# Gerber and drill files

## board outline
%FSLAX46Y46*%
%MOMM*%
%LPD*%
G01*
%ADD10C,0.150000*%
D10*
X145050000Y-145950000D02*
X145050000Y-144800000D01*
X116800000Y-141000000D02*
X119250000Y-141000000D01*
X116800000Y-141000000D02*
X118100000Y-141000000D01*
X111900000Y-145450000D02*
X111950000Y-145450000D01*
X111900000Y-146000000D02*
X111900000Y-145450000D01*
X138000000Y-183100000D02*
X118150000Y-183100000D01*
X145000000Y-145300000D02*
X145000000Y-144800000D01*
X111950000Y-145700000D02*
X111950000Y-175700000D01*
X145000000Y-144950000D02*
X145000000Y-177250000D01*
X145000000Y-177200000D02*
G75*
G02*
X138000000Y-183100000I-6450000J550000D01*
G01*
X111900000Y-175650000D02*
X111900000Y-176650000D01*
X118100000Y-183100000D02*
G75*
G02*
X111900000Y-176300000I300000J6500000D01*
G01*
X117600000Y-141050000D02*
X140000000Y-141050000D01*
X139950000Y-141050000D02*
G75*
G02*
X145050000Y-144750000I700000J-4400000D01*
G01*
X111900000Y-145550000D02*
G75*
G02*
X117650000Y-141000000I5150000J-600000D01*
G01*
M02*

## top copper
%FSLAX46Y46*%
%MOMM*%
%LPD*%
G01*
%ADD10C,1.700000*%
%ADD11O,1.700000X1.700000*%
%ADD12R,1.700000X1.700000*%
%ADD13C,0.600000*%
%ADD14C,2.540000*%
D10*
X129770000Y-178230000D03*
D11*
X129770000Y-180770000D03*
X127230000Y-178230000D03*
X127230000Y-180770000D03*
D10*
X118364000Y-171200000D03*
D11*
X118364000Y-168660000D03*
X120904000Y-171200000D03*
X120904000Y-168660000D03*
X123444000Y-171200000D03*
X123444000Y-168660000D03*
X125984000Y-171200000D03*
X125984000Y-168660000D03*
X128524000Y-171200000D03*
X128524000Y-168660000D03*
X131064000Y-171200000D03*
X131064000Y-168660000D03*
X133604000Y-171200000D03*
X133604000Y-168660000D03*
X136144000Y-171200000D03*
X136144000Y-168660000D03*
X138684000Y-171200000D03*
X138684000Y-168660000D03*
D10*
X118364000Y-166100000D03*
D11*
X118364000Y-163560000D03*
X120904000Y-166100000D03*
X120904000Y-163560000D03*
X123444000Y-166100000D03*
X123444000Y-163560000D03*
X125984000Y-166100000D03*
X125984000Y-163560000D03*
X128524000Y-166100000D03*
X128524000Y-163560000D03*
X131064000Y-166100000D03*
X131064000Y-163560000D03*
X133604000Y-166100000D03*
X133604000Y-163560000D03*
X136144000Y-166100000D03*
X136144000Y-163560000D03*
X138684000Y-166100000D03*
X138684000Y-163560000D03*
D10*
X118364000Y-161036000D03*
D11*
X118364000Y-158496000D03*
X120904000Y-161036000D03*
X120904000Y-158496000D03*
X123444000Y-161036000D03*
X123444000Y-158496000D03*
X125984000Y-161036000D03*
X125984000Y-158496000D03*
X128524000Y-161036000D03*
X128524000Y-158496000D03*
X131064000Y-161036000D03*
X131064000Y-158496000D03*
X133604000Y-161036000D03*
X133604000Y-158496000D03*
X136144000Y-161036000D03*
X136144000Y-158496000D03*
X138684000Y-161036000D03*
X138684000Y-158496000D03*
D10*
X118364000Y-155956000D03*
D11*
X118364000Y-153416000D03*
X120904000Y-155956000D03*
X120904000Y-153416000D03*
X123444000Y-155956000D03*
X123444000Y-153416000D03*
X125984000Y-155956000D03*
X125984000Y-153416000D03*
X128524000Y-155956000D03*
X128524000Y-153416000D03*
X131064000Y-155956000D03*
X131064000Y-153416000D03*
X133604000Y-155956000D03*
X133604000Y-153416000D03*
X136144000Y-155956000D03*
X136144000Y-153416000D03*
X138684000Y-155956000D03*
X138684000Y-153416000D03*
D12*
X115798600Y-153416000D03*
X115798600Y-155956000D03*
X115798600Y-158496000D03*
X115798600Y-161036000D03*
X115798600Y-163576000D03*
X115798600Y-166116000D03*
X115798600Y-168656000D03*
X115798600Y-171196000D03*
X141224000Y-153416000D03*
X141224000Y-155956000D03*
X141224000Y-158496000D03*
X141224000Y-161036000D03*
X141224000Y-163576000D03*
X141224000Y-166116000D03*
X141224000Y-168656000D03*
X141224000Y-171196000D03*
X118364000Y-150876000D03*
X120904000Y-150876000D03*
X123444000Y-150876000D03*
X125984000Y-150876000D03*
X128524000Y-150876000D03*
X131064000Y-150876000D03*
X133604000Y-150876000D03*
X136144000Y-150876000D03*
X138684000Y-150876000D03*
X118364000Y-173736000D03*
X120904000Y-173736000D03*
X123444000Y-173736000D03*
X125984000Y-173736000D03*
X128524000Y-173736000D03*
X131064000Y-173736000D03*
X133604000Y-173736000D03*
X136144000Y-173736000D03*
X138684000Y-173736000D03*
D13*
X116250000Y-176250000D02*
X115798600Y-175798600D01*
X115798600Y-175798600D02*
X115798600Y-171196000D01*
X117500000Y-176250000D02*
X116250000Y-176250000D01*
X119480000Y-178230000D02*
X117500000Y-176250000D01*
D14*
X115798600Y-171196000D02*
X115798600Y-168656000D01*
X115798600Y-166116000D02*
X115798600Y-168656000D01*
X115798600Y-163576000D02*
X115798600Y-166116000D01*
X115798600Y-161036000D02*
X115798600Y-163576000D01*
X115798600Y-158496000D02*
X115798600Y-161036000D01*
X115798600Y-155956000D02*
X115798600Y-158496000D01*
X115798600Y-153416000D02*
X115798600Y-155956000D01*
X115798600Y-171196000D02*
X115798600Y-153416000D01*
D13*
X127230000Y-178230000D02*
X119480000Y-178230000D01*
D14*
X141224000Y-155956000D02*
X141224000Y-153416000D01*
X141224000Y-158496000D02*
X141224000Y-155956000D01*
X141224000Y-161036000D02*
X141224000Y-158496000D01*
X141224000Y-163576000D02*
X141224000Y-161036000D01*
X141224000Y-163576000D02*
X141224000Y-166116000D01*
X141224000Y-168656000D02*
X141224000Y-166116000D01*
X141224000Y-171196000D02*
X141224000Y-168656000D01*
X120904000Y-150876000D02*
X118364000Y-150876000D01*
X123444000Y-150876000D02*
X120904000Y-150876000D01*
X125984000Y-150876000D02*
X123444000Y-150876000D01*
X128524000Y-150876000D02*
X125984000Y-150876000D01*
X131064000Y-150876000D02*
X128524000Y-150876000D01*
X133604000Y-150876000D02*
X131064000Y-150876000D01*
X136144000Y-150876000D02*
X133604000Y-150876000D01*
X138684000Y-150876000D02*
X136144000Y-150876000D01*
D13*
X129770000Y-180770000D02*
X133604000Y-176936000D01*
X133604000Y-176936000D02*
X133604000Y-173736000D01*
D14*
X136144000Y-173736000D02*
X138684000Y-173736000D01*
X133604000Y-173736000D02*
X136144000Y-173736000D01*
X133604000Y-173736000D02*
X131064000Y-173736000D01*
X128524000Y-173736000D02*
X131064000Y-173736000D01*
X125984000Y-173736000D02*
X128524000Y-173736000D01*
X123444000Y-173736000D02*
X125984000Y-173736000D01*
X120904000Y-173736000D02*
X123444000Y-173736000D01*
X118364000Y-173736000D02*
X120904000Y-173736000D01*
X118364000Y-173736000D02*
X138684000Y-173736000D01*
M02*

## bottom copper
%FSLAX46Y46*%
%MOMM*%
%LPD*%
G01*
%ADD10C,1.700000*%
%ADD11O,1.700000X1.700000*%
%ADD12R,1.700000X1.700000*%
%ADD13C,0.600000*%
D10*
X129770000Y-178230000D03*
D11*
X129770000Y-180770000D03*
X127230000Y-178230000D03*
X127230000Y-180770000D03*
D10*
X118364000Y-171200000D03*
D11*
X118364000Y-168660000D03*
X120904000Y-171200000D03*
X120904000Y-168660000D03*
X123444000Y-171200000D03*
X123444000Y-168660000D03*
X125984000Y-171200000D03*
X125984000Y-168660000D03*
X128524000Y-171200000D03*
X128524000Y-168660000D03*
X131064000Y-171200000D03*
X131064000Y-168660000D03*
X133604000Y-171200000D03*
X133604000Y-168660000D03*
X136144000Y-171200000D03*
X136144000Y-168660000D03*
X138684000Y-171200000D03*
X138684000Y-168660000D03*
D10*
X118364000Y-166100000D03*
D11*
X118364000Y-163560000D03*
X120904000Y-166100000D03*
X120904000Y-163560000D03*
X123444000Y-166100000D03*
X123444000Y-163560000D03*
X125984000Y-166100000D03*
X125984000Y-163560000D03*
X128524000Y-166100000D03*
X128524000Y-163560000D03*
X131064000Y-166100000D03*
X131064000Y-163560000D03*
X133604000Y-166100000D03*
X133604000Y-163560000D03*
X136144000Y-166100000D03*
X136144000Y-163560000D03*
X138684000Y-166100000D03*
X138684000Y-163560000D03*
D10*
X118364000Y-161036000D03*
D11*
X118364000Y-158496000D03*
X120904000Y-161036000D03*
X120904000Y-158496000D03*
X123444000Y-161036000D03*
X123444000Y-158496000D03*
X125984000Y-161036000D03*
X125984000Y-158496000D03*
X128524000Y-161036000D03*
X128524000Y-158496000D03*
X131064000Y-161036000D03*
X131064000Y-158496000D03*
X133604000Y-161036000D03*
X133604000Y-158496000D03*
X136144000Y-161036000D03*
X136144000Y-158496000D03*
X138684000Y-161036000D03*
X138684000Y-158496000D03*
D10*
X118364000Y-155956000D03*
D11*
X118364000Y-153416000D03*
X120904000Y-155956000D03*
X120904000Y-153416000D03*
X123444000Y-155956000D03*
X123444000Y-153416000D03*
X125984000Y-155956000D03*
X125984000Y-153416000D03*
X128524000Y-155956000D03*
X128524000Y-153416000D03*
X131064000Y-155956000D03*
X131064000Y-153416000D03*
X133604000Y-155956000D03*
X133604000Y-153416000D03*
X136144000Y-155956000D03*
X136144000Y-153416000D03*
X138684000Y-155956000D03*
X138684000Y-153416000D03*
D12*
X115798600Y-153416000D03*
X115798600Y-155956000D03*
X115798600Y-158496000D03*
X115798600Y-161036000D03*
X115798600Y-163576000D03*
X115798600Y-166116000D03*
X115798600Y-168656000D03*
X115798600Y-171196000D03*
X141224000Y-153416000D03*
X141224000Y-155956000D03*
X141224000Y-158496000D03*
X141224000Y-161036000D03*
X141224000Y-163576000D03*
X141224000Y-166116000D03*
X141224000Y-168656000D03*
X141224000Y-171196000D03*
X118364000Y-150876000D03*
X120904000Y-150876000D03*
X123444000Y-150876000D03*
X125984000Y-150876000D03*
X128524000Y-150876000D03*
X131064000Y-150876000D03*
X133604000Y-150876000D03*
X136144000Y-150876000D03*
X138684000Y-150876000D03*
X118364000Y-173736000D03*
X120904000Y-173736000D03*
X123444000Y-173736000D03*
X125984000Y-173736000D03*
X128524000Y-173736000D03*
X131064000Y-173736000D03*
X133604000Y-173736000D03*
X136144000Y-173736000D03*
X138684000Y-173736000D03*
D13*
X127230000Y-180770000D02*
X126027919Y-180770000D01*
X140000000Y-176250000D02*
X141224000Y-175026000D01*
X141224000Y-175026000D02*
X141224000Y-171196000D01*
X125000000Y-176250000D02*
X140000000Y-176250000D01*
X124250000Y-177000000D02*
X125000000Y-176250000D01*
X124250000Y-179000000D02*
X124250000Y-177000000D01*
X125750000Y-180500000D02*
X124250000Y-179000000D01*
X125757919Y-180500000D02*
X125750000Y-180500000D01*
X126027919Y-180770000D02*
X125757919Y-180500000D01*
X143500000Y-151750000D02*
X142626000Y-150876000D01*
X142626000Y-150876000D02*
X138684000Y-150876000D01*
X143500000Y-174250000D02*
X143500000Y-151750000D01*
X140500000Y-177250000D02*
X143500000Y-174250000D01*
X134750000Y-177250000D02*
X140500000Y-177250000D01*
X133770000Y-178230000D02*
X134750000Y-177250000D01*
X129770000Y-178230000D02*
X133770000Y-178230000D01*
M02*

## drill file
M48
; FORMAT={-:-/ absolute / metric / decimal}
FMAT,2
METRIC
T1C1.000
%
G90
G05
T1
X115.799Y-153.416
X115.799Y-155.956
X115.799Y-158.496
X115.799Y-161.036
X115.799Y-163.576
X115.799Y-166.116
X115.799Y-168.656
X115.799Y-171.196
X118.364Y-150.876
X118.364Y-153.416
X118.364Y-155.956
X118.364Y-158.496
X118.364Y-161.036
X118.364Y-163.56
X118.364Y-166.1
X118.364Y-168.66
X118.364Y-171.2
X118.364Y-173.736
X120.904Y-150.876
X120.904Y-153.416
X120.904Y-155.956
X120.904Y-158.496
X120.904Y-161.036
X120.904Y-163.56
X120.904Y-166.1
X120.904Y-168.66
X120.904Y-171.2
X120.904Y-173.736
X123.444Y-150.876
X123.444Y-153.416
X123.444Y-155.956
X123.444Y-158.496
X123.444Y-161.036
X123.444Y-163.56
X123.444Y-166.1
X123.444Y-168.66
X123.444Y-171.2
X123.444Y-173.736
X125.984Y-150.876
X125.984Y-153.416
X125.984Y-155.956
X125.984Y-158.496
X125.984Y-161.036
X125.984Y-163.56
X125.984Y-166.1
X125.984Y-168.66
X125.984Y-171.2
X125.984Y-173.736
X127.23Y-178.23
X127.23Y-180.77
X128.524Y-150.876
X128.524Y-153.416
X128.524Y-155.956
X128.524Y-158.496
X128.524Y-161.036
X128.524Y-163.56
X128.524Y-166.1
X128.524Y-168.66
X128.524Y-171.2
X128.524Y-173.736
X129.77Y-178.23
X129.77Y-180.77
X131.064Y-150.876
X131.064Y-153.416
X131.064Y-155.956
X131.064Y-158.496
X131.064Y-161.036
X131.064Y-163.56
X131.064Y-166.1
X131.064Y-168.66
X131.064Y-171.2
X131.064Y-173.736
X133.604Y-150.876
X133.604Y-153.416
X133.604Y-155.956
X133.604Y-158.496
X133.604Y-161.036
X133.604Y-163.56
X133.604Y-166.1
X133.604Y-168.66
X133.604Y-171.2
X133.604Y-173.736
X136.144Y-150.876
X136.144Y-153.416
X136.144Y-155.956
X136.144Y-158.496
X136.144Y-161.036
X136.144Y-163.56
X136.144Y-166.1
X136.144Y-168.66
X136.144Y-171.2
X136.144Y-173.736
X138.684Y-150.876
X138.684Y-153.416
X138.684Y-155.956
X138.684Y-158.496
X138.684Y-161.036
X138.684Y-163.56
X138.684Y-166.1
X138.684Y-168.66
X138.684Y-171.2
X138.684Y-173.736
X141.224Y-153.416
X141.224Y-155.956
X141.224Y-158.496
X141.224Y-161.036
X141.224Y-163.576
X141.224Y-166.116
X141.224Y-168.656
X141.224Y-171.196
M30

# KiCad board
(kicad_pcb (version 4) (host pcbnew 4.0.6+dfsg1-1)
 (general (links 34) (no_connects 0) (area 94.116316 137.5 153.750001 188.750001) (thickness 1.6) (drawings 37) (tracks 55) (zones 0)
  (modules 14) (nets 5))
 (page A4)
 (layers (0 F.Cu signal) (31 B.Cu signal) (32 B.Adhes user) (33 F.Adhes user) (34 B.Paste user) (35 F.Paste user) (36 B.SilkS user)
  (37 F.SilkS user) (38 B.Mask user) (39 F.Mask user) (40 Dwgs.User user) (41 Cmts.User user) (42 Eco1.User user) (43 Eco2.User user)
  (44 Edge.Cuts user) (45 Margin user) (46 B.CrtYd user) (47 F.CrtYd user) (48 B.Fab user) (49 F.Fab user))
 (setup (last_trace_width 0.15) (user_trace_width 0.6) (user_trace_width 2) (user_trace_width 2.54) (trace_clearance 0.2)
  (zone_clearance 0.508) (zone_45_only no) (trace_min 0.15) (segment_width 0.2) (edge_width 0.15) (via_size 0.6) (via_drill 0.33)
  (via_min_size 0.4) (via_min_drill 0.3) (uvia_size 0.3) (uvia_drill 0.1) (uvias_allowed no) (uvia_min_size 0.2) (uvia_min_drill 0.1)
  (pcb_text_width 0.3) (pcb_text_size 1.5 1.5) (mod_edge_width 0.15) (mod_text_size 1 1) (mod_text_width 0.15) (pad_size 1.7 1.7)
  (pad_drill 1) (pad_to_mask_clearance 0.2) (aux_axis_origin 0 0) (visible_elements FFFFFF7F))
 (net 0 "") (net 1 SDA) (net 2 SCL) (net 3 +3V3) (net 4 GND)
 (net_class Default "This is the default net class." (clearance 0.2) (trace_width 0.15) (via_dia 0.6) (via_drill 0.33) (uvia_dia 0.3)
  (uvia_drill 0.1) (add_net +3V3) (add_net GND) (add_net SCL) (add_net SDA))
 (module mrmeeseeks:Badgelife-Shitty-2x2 (layer F.Cu) (at 128.5 179.5)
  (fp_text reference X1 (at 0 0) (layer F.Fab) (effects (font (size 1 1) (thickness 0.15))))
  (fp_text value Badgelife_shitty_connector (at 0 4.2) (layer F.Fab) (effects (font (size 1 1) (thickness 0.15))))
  (pad 4 thru_hole circle (at 1.27 -1.27) (size 1.7 1.7) (drill 1) (layers *.Cu *.Mask) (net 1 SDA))
  (pad 3 thru_hole oval (at 1.27 1.27) (size 1.7 1.7) (drill 1) (layers *.Cu *.Mask) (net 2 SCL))
  (pad 1 thru_hole oval (at -1.27 -1.27) (size 1.7 1.7) (drill 1) (layers *.Cu *.Mask) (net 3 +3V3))
  (pad 2 thru_hole oval (at -1.27 1.27) (size 1.7 1.7) (drill 1) (layers *.Cu *.Mask) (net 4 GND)))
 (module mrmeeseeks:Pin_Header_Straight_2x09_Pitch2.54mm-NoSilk (layer F.Cu) (at 118.364 171.2 90)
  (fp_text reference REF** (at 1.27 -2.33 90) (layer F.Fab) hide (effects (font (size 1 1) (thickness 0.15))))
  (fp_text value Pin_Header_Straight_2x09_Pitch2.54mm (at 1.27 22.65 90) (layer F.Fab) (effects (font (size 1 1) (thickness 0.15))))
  (pad 1 thru_hole circle (at 0 0 90) (size 1.7 1.7) (drill 1) (layers *.Cu *.Mask))
  (pad 2 thru_hole oval (at 2.54 0 90) (size 1.7 1.7) (drill 1) (layers *.Cu *.Mask))
  (pad 3 thru_hole oval (at 0 2.54 90) (size 1.7 1.7) (drill 1) (layers *.Cu *.Mask))
  (pad 4 thru_hole oval (at 2.54 2.54 90) (size 1.7 1.7) (drill 1) (layers *.Cu *.Mask))
  (pad 5 thru_hole oval (at 0 5.08 90) (size 1.7 1.7) (drill 1) (layers *.Cu *.Mask))
  (pad 6 thru_hole oval (at 2.54 5.08 90) (size 1.7 1.7) (drill 1) (layers *.Cu *.Mask))
  (pad 7 thru_hole oval (at 0 7.62 90) (size 1.7 1.7) (drill 1) (layers *.Cu *.Mask))
  (pad 8 thru_hole oval (at 2.54 7.62 90) (size 1.7 1.7) (drill 1) (layers *.Cu *.Mask))
  (pad 9 thru_hole oval (at 0 10.16 90) (size 1.7 1.7) (drill 1) (layers *.Cu *.Mask))
  (pad 10 thru_hole oval (at 2.54 10.16 90) (size 1.7 1.7) (drill 1) (layers *.Cu *.Mask))
  (pad 11 thru_hole oval (at 0 12.7 90) (size 1.7 1.7) (drill 1) (layers *.Cu *.Mask))
  (pad 12 thru_hole oval (at 2.54 12.7 90) (size 1.7 1.7) (drill 1) (layers *.Cu *.Mask))
  (pad 13 thru_hole oval (at 0 15.24 90) (size 1.7 1.7) (drill 1) (layers *.Cu *.Mask))
  (pad 14 thru_hole oval (at 2.54 15.24 90) (size 1.7 1.7) (drill 1) (layers *.Cu *.Mask))
  (pad 15 thru_hole oval (at 0 17.78 90) (size 1.7 1.7) (drill 1) (layers *.Cu *.Mask))
  (pad 16 thru_hole oval (at 2.54 17.78 90) (size 1.7 1.7) (drill 1) (layers *.Cu *.Mask))
  (pad 17 thru_hole oval (at 0 20.32 90) (size 1.7 1.7) (drill 1) (layers *.Cu *.Mask))
  (pad 18 thru_hole oval (at 2.54 20.32 90) (size 1.7 1.7) (drill 1) (layers *.Cu *.Mask)))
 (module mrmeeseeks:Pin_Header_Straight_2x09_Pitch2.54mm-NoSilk (layer F.Cu) (at 118.364 166.1 90)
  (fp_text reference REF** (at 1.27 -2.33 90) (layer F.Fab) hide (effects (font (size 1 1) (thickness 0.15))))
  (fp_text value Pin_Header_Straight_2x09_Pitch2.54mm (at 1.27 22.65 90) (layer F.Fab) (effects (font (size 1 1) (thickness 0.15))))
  (pad 1 thru_hole circle (at 0 0 90) (size 1.7 1.7) (drill 1) (layers *.Cu *.Mask))
  (pad 2 thru_hole oval (at 2.54 0 90) (size 1.7 1.7) (drill 1) (layers *.Cu *.Mask))
  (pad 3 thru_hole oval (at 0 2.54 90) (size 1.7 1.7) (drill 1) (layers *.Cu *.Mask))
  (pad 4 thru_hole oval (at 2.54 2.54 90) (size 1.7 1.7) (drill 1) (layers *.Cu *.Mask))
  (pad 5 thru_hole oval (at 0 5.08 90) (size 1.7 1.7) (drill 1) (layers *.Cu *.Mask))
  (pad 6 thru_hole oval (at 2.54 5.08 90) (size 1.7 1.7) (drill 1) (layers *.Cu *.Mask))
  (pad 7 thru_hole oval (at 0 7.62 90) (size 1.7 1.7) (drill 1) (layers *.Cu *.Mask))
  (pad 8 thru_hole oval (at 2.54 7.62 90) (size 1.7 1.7) (drill 1) (layers *.Cu *.Mask))
  (pad 9 thru_hole oval (at 0 10.16 90) (size 1.7 1.7) (drill 1) (layers *.Cu *.Mask))
  (pad 10 thru_hole oval (at 2.54 10.16 90) (size 1.7 1.7) (drill 1) (layers *.Cu *.Mask))
  (pad 11 thru_hole oval (at 0 12.7 90) (size 1.7 1.7) (drill 1) (layers *.Cu *.Mask))
  (pad 12 thru_hole oval (at 2.54 12.7 90) (size 1.7 1.7) (drill 1) (layers *.Cu *.Mask))
  (pad 13 thru_hole oval (at 0 15.24 90) (size 1.7 1.7) (drill 1) (layers *.Cu *.Mask))
  (pad 14 thru_hole oval (at 2.54 15.24 90) (size 1.7 1.7) (drill 1) (layers *.Cu *.Mask))
  (pad 15 thru_hole oval (at 0 17.78 90) (size 1.7 1.7) (drill 1) (layers *.Cu *.Mask))
  (pad 16 thru_hole oval (at 2.54 17.78 90) (size 1.7 1.7) (drill 1) (layers *.Cu *.Mask))
  (pad 17 thru_hole oval (at 0 20.32 90) (size 1.7 1.7) (drill 1) (layers *.Cu *.Mask))
  (pad 18 thru_hole oval (at 2.54 20.32 90) (size 1.7 1.7) (drill 1) (layers *.Cu *.Mask)))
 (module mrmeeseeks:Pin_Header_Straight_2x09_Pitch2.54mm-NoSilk (layer F.Cu) (at 118.364 161.036 90)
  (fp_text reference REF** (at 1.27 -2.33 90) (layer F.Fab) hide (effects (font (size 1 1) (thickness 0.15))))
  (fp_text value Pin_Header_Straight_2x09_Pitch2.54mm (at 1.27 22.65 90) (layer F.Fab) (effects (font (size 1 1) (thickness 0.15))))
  (pad 1 thru_hole circle (at 0 0 90) (size 1.7 1.7) (drill 1) (layers *.Cu *.Mask))
  (pad 2 thru_hole oval (at 2.54 0 90) (size 1.7 1.7) (drill 1) (layers *.Cu *.Mask))
  (pad 3 thru_hole oval (at 0 2.54 90) (size 1.7 1.7) (drill 1) (layers *.Cu *.Mask))
  (pad 4 thru_hole oval (at 2.54 2.54 90) (size 1.7 1.7) (drill 1) (layers *.Cu *.Mask))
  (pad 5 thru_hole oval (at 0 5.08 90) (size 1.7 1.7) (drill 1) (layers *.Cu *.Mask))
  (pad 6 thru_hole oval (at 2.54 5.08 90) (size 1.7 1.7) (drill 1) (layers *.Cu *.Mask))
  (pad 7 thru_hole oval (at 0 7.62 90) (size 1.7 1.7) (drill 1) (layers *.Cu *.Mask))
  (pad 8 thru_hole oval (at 2.54 7.62 90) (size 1.7 1.7) (drill 1) (layers *.Cu *.Mask))
  (pad 9 thru_hole oval (at 0 10.16 90) (size 1.7 1.7) (drill 1) (layers *.Cu *.Mask))
  (pad 10 thru_hole oval (at 2.54 10.16 90) (size 1.7 1.7) (drill 1) (layers *.Cu *.Mask))
  (pad 11 thru_hole oval (at 0 12.7 90) (size 1.7 1.7) (drill 1) (layers *.Cu *.Mask))
  (pad 12 thru_hole oval (at 2.54 12.7 90) (size 1.7 1.7) (drill 1) (layers *.Cu *.Mask))
  (pad 13 thru_hole oval (at 0 15.24 90) (size 1.7 1.7) (drill 1) (layers *.Cu *.Mask))
  (pad 14 thru_hole oval (at 2.54 15.24 90) (size 1.7 1.7) (drill 1) (layers *.Cu *.Mask))
  (pad 15 thru_hole oval (at 0 17.78 90) (size 1.7 1.7) (drill 1) (layers *.Cu *.Mask))
  (pad 16 thru_hole oval (at 2.54 17.78 90) (size 1.7 1.7) (drill 1) (layers *.Cu *.Mask))
  (pad 17 thru_hole oval (at 0 20.32 90) (size 1.7 1.7) (drill 1) (layers *.Cu *.Mask))
  (pad 18 thru_hole oval (at 2.54 20.32 90) (size 1.7 1.7) (drill 1) (layers *.Cu *.Mask)))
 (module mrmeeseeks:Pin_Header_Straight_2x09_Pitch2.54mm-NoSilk (layer F.Cu) (at 118.364 155.956 90)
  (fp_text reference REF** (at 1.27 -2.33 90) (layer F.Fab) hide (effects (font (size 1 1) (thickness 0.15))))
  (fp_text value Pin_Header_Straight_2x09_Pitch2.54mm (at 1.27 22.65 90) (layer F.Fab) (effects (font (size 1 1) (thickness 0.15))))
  (pad 1 thru_hole circle (at 0 0 90) (size 1.7 1.7) (drill 1) (layers *.Cu *.Mask))
  (pad 2 thru_hole oval (at 2.54 0 90) (size 1.7 1.7) (drill 1) (layers *.Cu *.Mask))
  (pad 3 thru_hole oval (at 0 2.54 90) (size 1.7 1.7) (drill 1) (layers *.Cu *.Mask))
  (pad 4 thru_hole oval (at 2.54 2.54 90) (size 1.7 1.7) (drill 1) (layers *.Cu *.Mask))
  (pad 5 thru_hole oval (at 0 5.08 90) (size 1.7 1.7) (drill 1) (layers *.Cu *.Mask))
  (pad 6 thru_hole oval (at 2.54 5.08 90) (size 1.7 1.7) (drill 1) (layers *.Cu *.Mask))
  (pad 7 thru_hole oval (at 0 7.62 90) (size 1.7 1.7) (drill 1) (layers *.Cu *.Mask))
  (pad 8 thru_hole oval (at 2.54 7.62 90) (size 1.7 1.7) (drill 1) (layers *.Cu *.Mask))
  (pad 9 thru_hole oval (at 0 10.16 90) (size 1.7 1.7) (drill 1) (layers *.Cu *.Mask))
  (pad 10 thru_hole oval (at 2.54 10.16 90) (size 1.7 1.7) (drill 1) (layers *.Cu *.Mask))
  (pad 11 thru_hole oval (at 0 12.7 90) (size 1.7 1.7) (drill 1) (layers *.Cu *.Mask))
  (pad 12 thru_hole oval (at 2.54 12.7 90) (size 1.7 1.7) (drill 1) (layers *.Cu *.Mask))
  (pad 13 thru_hole oval (at 0 15.24 90) (size 1.7 1.7) (drill 1) (layers *.Cu *.Mask))
  (pad 14 thru_hole oval (at 2.54 15.24 90) (size 1.7 1.7) (drill 1) (layers *.Cu *.Mask))
  (pad 15 thru_hole oval (at 0 17.78 90) (size 1.7 1.7) (drill 1) (layers *.Cu *.Mask))
  (pad 16 thru_hole oval (at 2.54 17.78 90) (size 1.7 1.7) (drill 1) (layers *.Cu *.Mask))
  (pad 17 thru_hole oval (at 0 20.32 90) (size 1.7 1.7) (drill 1) (layers *.Cu *.Mask))
  (pad 18 thru_hole oval (at 2.54 20.32 90) (size 1.7 1.7) (drill 1) (layers *.Cu *.Mask)))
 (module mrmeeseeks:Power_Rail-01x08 (layer F.Cu) (at 115.7986 153.416)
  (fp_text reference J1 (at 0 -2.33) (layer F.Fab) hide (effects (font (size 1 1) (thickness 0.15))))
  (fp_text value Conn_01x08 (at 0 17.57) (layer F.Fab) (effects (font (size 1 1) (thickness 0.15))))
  (pad 1 thru_hole rect (at 0 0) (size 1.7 1.7) (drill 1) (layers *.Cu *.Mask) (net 3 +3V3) (solder_mask_margin 0.1))
  (pad 2 thru_hole rect (at 0 2.54) (size 1.7 1.7) (drill 1) (layers *.Cu *.Mask) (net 3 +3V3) (solder_mask_margin 0.1))
  (pad 3 thru_hole rect (at 0 5.08) (size 1.7 1.7) (drill 1) (layers *.Cu *.Mask) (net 3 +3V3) (solder_mask_margin 0.1))
  (pad 4 thru_hole rect (at 0 7.62) (size 1.7 1.7) (drill 1) (layers *.Cu *.Mask) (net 3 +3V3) (solder_mask_margin 0.1))
  (pad 5 thru_hole rect (at 0 10.16) (size 1.7 1.7) (drill 1) (layers *.Cu *.Mask) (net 3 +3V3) (solder_mask_margin 0.1))
  (pad 6 thru_hole rect (at 0 12.7) (size 1.7 1.7) (drill 1) (layers *.Cu *.Mask) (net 3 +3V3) (solder_mask_margin 0.1))
  (pad 7 thru_hole rect (at 0 15.24) (size 1.7 1.7) (drill 1) (layers *.Cu *.Mask) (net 3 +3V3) (solder_mask_margin 0.1))
  (pad 8 thru_hole rect (at 0 17.78) (size 1.7 1.7) (drill 1) (layers *.Cu *.Mask) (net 3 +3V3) (solder_mask_margin 0.1)))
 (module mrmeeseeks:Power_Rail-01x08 (layer F.Cu) (at 141.224 153.416)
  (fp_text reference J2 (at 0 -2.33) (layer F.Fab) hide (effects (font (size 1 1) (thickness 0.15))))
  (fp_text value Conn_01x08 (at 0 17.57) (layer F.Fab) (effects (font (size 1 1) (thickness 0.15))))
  (pad 1 thru_hole rect (at 0 0) (size 1.7 1.7) (drill 1) (layers *.Cu *.Mask) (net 4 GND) (solder_mask_margin 0.1))
  (pad 2 thru_hole rect (at 0 2.54) (size 1.7 1.7) (drill 1) (layers *.Cu *.Mask) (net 4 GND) (solder_mask_margin 0.1))
  (pad 3 thru_hole rect (at 0 5.08) (size 1.7 1.7) (drill 1) (layers *.Cu *.Mask) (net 4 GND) (solder_mask_margin 0.1))
  (pad 4 thru_hole rect (at 0 7.62) (size 1.7 1.7) (drill 1) (layers *.Cu *.Mask) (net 4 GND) (solder_mask_margin 0.1))
  (pad 5 thru_hole rect (at 0 10.16) (size 1.7 1.7) (drill 1) (layers *.Cu *.Mask) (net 4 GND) (solder_mask_margin 0.1))
  (pad 6 thru_hole rect (at 0 12.7) (size 1.7 1.7) (drill 1) (layers *.Cu *.Mask) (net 4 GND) (solder_mask_margin 0.1))
  (pad 7 thru_hole rect (at 0 15.24) (size 1.7 1.7) (drill 1) (layers *.Cu *.Mask) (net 4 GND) (solder_mask_margin 0.1))
  (pad 8 thru_hole rect (at 0 17.78) (size 1.7 1.7) (drill 1) (layers *.Cu *.Mask) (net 4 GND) (solder_mask_margin 0.1)))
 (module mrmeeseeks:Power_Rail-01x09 (layer F.Cu) (at 118.364 150.876 90)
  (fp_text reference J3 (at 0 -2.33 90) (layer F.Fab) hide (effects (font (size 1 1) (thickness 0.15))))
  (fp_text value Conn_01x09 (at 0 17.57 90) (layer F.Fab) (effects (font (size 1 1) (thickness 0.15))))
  (pad 1 thru_hole rect (at 0 0 90) (size 1.7 1.7) (drill 1) (layers *.Cu *.Mask) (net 1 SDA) (solder_mask_margin 0.1))
  (pad 2 thru_hole rect (at 0 2.54 90) (size 1.7 1.7) (drill 1) (layers *.Cu *.Mask) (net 1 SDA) (solder_mask_margin 0.1))
  (pad 3 thru_hole rect (at 0 5.08 90) (size 1.7 1.7) (drill 1) (layers *.Cu *.Mask) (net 1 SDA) (solder_mask_margin 0.1))
  (pad 4 thru_hole rect (at 0 7.62 90) (size 1.7 1.7) (drill 1) (layers *.Cu *.Mask) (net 1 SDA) (solder_mask_margin 0.1))
  (pad 5 thru_hole rect (at 0 10.16 90) (size 1.7 1.7) (drill 1) (layers *.Cu *.Mask) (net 1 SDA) (solder_mask_margin 0.1))
  (pad 6 thru_hole rect (at 0 12.7 90) (size 1.7 1.7) (drill 1) (layers *.Cu *.Mask) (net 1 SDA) (solder_mask_margin 0.1))
  (pad 7 thru_hole rect (at 0 15.24 90) (size 1.7 1.7) (drill 1) (layers *.Cu *.Mask) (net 1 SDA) (solder_mask_margin 0.1))
  (pad 8 thru_hole rect (at 0 17.78 90) (size 1.7 1.7) (drill 1) (layers *.Cu *.Mask) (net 1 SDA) (solder_mask_margin 0.1))
  (pad 9 thru_hole rect (at 0 20.32 90) (size 1.7 1.7) (drill 1) (layers *.Cu *.Mask) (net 1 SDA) (solder_mask_margin 0.1)))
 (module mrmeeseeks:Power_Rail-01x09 (layer F.Cu) (at 118.364 173.736 90)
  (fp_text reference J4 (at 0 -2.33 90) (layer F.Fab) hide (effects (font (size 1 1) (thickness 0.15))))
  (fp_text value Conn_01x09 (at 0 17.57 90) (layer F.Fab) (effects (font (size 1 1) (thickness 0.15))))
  (pad 1 thru_hole rect (at 0 0 90) (size 1.7 1.7) (drill 1) (layers *.Cu *.Mask) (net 2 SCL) (solder_mask_margin 0.1))
  (pad 2 thru_hole rect (at 0 2.54 90) (size 1.7 1.7) (drill 1) (layers *.Cu *.Mask) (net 2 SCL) (solder_mask_margin 0.1))
  (pad 3 thru_hole rect (at 0 5.08 90) (size 1.7 1.7) (drill 1) (layers *.Cu *.Mask) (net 2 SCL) (solder_mask_margin 0.1))
  (pad 4 thru_hole rect (at 0 7.62 90) (size 1.7 1.7) (drill 1) (layers *.Cu *.Mask) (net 2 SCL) (solder_mask_margin 0.1))
  (pad 5 thru_hole rect (at 0 10.16 90) (size 1.7 1.7) (drill 1) (layers *.Cu *.Mask) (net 2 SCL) (solder_mask_margin 0.1))
  (pad 6 thru_hole rect (at 0 12.7 90) (size 1.7 1.7) (drill 1) (layers *.Cu *.Mask) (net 2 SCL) (solder_mask_margin 0.1))
  (pad 7 thru_hole rect (at 0 15.24 90) (size 1.7 1.7) (drill 1) (layers *.Cu *.Mask) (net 2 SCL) (solder_mask_margin 0.1))
  (pad 8 thru_hole rect (at 0 17.78 90) (size 1.7 1.7) (drill 1) (layers *.Cu *.Mask) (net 2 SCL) (solder_mask_margin 0.1))
  (pad 9 thru_hole rect (at 0 20.32 90) (size 1.7 1.7) (drill 1) (layers *.Cu *.Mask) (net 2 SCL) (solder_mask_margin 0.1)))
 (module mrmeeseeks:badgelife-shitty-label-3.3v (layer F.Cu) (at 113.4 162.2 90)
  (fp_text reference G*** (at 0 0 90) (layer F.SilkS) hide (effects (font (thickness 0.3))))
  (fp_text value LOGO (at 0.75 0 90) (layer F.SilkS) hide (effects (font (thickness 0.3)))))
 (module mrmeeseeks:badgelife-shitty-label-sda (layer F.Cu) (at 128.2 148.8)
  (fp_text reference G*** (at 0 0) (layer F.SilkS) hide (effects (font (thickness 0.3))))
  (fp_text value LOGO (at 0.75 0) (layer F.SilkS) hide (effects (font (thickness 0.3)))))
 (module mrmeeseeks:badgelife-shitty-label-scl (layer F.Cu) (at 128.4 175.7)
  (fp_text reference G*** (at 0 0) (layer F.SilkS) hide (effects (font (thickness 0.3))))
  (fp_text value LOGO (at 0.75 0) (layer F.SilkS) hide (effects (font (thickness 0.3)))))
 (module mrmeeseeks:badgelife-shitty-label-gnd (layer F.Cu) (at 143.7 162.3 270)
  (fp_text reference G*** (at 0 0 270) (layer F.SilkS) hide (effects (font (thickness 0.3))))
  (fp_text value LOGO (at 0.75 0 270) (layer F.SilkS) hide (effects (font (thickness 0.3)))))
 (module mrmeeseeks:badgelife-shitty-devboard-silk (layer F.Cu) (at 128.9 144.6)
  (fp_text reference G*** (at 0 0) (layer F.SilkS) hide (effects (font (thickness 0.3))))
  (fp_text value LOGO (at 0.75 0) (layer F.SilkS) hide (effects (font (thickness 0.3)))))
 (gr_line (start 145.05 145.95) (end 145.05 144.8) (angle 90) (layer Edge.Cuts) (width 0.15))
 (gr_line (start 116.8 141) (end 119.25 141) (angle 90) (layer Edge.Cuts) (width 0.15))
 (gr_line (start 116.8 141) (end 118.1 141) (angle 90) (layer Edge.Cuts) (width 0.15))
 (gr_line (start 111.9 145.45) (end 111.95 145.45) (angle 90) (layer Edge.Cuts) (width 0.15))
 (gr_line (start 111.9 146) (end 111.9 145.45) (angle 90) (layer Edge.Cuts) (width 0.15))
 (gr_line (start 138 183.1) (end 118.15 183.1) (angle 90) (layer Edge.Cuts) (width 0.15))
 (gr_line (start 145 145.3) (end 145 144.8) (angle 90) (layer Edge.Cuts) (width 0.15))
 (gr_line (start 111.95 145.7) (end 111.95 175.7) (angle 90) (layer Edge.Cuts) (width 0.15))
 (gr_line (start 145 144.95) (end 145 177.25) (angle 90) (layer Edge.Cuts) (width 0.15))
 (gr_arc (start 138.55 176.65) (end 145 177.2) (angle 90) (layer Edge.Cuts) (width 0.15))
 (gr_line (start 111.9 175.65) (end 111.9 176.65) (angle 90) (layer Edge.Cuts) (width 0.15))
 (gr_arc (start 118.4 176.6) (end 118.1 183.1) (angle 90) (layer Edge.Cuts) (width 0.15))
 (gr_line (start 117.6 141.05) (end 140 141.05) (angle 90) (layer Edge.Cuts) (width 0.15))
 (gr_arc (start 140.65 145.45) (end 139.95 141.05) (angle 90) (layer Edge.Cuts) (width 0.15))
 (gr_arc (start 117.05 146.15) (end 111.9 145.55) (angle 90) (layer Edge.Cuts) (width 0.15))
 (segment (start 116.25 176.25) (end 115.7986 175.7986) (width 0.6) (layer F.Cu) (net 3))
 (segment (start 115.7986 175.7986) (end 115.7986 171.196) (width 0.6) (layer F.Cu) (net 3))
 (segment (start 117.5 176.25) (end 116.25 176.25) (width 0.6) (layer F.Cu) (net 3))
 (segment (start 119.48 178.23) (end 117.5 176.25) (width 0.6) (layer F.Cu) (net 3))
 (segment (start 115.7986 171.196) (end 115.7986 168.656) (width 2.54) (layer F.Cu) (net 3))
 (segment (start 115.7986 166.116) (end 115.7986 168.656) (width 2.54) (layer F.Cu) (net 3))
 (segment (start 115.7986 163.576) (end 115.7986 166.116) (width 2.54) (layer F.Cu) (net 3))
 (segment (start 115.7986 161.036) (end 115.7986 163.576) (width 2.54) (layer F.Cu) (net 3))
 (segment (start 115.7986 158.496) (end 115.7986 161.036) (width 2.54) (layer F.Cu) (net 3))
 (segment (start 115.7986 155.956) (end 115.7986 158.496) (width 2.54) (layer F.Cu) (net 3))
 (segment (start 115.7986 153.416) (end 115.7986 155.956) (width 2.54) (layer F.Cu) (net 3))
 (segment (start 115.7986 171.196) (end 115.7986 153.416) (width 2.54) (layer F.Cu) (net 3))
 (segment (start 127.23 178.23) (end 119.48 178.23) (width 0.6) (layer F.Cu) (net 3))
 (segment (start 127.23 180.77) (end 126.027919 180.77) (width 0.6) (layer B.Cu) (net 4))
 (segment (start 140 176.25) (end 141.224 175.026) (width 0.6) (layer B.Cu) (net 4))
 (segment (start 141.224 175.026) (end 141.224 171.196) (width 0.6) (layer B.Cu) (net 4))
 (segment (start 125 176.25) (end 140 176.25) (width 0.6) (layer B.Cu) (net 4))
 (segment (start 124.25 177) (end 125 176.25) (width 0.6) (layer B.Cu) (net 4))
 (segment (start 124.25 179) (end 124.25 177) (width 0.6) (layer B.Cu) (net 4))
 (segment (start 125.75 180.5) (end 124.25 179) (width 0.6) (layer B.Cu) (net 4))
 (segment (start 125.757919 180.5) (end 125.75 180.5) (width 0.6) (layer B.Cu) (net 4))
 (segment (start 126.027919 180.77) (end 125.757919 180.5) (width 0.6) (layer B.Cu) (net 4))
 (segment (start 141.224 155.956) (end 141.224 153.416) (width 2.54) (layer F.Cu) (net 4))
 (segment (start 141.224 158.496) (end 141.224 155.956) (width 2.54) (layer F.Cu) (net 4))
 (segment (start 141.224 161.036) (end 141.224 158.496) (width 2.54) (layer F.Cu) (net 4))
 (segment (start 141.224 163.576) (end 141.224 161.036) (width 2.54) (layer F.Cu) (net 4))
 (segment (start 141.224 163.576) (end 141.224 166.116) (width 2.54) (layer F.Cu) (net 4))
 (segment (start 141.224 168.656) (end 141.224 166.116) (width 2.54) (layer F.Cu) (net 4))
 (segment (start 141.224 171.196) (end 141.224 168.656) (width 2.54) (layer F.Cu) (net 4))
 (segment (start 143.5 151.75) (end 142.626 150.876) (width 0.6) (layer B.Cu) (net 1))
 (segment (start 142.626 150.876) (end 138.684 150.876) (width 0.6) (layer B.Cu) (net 1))
 (segment (start 143.5 174.25) (end 143.5 151.75) (width 0.6) (layer B.Cu) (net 1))
 (segment (start 140.5 177.25) (end 143.5 174.25) (width 0.6) (layer B.Cu) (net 1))
 (segment (start 134.75 177.25) (end 140.5 177.25) (width 0.6) (layer B.Cu) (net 1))
 (segment (start 133.77 178.23) (end 134.75 177.25) (width 0.6) (layer B.Cu) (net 1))
 (segment (start 120.904 150.876) (end 118.364 150.876) (width 2.54) (layer F.Cu) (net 1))
 (segment (start 123.444 150.876) (end 120.904 150.876) (width 2.54) (layer F.Cu) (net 1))
 (segment (start 125.984 150.876) (end 123.444 150.876) (width 2.54) (layer F.Cu) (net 1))
 (segment (start 128.524 150.876) (end 125.984 150.876) (width 2.54) (layer F.Cu) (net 1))
 (segment (start 131.064 150.876) (end 128.524 150.876) (width 2.54) (layer F.Cu) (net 1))
 (segment (start 133.604 150.876) (end 131.064 150.876) (width 2.54) (layer F.Cu) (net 1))
 (segment (start 136.144 150.876) (end 133.604 150.876) (width 2.54) (layer F.Cu) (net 1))
 (segment (start 138.684 150.876) (end 136.144 150.876) (width 2.54) (layer F.Cu) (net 1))
 (segment (start 129.77 178.23) (end 133.77 178.23) (width 0.6) (layer B.Cu) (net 1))
 (segment (start 129.77 180.77) (end 133.604 176.936) (width 0.6) (layer F.Cu) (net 2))
 (segment (start 133.604 176.936) (end 133.604 173.736) (width 0.6) (layer F.Cu) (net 2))
 (segment (start 136.144 173.736) (end 138.684 173.736) (width 2.54) (layer F.Cu) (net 2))
 (segment (start 133.604 173.736) (end 136.144 173.736) (width 2.54) (layer F.Cu) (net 2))
 (segment (start 133.604 173.736) (end 131.064 173.736) (width 2.54) (layer F.Cu) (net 2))
 (segment (start 128.524 173.736) (end 131.064 173.736) (width 2.54) (layer F.Cu) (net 2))
 (segment (start 125.984 173.736) (end 128.524 173.736) (width 2.54) (layer F.Cu) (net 2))
 (segment (start 123.444 173.736) (end 125.984 173.736) (width 2.54) (layer F.Cu) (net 2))
 (segment (start 120.904 173.736) (end 123.444 173.736) (width 2.54) (layer F.Cu) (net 2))
 (segment (start 118.364 173.736) (end 120.904 173.736) (width 2.54) (layer F.Cu) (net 2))
 (segment (start 118.364 173.736) (end 138.684 173.736) (width 2.54) (layer F.Cu) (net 2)))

